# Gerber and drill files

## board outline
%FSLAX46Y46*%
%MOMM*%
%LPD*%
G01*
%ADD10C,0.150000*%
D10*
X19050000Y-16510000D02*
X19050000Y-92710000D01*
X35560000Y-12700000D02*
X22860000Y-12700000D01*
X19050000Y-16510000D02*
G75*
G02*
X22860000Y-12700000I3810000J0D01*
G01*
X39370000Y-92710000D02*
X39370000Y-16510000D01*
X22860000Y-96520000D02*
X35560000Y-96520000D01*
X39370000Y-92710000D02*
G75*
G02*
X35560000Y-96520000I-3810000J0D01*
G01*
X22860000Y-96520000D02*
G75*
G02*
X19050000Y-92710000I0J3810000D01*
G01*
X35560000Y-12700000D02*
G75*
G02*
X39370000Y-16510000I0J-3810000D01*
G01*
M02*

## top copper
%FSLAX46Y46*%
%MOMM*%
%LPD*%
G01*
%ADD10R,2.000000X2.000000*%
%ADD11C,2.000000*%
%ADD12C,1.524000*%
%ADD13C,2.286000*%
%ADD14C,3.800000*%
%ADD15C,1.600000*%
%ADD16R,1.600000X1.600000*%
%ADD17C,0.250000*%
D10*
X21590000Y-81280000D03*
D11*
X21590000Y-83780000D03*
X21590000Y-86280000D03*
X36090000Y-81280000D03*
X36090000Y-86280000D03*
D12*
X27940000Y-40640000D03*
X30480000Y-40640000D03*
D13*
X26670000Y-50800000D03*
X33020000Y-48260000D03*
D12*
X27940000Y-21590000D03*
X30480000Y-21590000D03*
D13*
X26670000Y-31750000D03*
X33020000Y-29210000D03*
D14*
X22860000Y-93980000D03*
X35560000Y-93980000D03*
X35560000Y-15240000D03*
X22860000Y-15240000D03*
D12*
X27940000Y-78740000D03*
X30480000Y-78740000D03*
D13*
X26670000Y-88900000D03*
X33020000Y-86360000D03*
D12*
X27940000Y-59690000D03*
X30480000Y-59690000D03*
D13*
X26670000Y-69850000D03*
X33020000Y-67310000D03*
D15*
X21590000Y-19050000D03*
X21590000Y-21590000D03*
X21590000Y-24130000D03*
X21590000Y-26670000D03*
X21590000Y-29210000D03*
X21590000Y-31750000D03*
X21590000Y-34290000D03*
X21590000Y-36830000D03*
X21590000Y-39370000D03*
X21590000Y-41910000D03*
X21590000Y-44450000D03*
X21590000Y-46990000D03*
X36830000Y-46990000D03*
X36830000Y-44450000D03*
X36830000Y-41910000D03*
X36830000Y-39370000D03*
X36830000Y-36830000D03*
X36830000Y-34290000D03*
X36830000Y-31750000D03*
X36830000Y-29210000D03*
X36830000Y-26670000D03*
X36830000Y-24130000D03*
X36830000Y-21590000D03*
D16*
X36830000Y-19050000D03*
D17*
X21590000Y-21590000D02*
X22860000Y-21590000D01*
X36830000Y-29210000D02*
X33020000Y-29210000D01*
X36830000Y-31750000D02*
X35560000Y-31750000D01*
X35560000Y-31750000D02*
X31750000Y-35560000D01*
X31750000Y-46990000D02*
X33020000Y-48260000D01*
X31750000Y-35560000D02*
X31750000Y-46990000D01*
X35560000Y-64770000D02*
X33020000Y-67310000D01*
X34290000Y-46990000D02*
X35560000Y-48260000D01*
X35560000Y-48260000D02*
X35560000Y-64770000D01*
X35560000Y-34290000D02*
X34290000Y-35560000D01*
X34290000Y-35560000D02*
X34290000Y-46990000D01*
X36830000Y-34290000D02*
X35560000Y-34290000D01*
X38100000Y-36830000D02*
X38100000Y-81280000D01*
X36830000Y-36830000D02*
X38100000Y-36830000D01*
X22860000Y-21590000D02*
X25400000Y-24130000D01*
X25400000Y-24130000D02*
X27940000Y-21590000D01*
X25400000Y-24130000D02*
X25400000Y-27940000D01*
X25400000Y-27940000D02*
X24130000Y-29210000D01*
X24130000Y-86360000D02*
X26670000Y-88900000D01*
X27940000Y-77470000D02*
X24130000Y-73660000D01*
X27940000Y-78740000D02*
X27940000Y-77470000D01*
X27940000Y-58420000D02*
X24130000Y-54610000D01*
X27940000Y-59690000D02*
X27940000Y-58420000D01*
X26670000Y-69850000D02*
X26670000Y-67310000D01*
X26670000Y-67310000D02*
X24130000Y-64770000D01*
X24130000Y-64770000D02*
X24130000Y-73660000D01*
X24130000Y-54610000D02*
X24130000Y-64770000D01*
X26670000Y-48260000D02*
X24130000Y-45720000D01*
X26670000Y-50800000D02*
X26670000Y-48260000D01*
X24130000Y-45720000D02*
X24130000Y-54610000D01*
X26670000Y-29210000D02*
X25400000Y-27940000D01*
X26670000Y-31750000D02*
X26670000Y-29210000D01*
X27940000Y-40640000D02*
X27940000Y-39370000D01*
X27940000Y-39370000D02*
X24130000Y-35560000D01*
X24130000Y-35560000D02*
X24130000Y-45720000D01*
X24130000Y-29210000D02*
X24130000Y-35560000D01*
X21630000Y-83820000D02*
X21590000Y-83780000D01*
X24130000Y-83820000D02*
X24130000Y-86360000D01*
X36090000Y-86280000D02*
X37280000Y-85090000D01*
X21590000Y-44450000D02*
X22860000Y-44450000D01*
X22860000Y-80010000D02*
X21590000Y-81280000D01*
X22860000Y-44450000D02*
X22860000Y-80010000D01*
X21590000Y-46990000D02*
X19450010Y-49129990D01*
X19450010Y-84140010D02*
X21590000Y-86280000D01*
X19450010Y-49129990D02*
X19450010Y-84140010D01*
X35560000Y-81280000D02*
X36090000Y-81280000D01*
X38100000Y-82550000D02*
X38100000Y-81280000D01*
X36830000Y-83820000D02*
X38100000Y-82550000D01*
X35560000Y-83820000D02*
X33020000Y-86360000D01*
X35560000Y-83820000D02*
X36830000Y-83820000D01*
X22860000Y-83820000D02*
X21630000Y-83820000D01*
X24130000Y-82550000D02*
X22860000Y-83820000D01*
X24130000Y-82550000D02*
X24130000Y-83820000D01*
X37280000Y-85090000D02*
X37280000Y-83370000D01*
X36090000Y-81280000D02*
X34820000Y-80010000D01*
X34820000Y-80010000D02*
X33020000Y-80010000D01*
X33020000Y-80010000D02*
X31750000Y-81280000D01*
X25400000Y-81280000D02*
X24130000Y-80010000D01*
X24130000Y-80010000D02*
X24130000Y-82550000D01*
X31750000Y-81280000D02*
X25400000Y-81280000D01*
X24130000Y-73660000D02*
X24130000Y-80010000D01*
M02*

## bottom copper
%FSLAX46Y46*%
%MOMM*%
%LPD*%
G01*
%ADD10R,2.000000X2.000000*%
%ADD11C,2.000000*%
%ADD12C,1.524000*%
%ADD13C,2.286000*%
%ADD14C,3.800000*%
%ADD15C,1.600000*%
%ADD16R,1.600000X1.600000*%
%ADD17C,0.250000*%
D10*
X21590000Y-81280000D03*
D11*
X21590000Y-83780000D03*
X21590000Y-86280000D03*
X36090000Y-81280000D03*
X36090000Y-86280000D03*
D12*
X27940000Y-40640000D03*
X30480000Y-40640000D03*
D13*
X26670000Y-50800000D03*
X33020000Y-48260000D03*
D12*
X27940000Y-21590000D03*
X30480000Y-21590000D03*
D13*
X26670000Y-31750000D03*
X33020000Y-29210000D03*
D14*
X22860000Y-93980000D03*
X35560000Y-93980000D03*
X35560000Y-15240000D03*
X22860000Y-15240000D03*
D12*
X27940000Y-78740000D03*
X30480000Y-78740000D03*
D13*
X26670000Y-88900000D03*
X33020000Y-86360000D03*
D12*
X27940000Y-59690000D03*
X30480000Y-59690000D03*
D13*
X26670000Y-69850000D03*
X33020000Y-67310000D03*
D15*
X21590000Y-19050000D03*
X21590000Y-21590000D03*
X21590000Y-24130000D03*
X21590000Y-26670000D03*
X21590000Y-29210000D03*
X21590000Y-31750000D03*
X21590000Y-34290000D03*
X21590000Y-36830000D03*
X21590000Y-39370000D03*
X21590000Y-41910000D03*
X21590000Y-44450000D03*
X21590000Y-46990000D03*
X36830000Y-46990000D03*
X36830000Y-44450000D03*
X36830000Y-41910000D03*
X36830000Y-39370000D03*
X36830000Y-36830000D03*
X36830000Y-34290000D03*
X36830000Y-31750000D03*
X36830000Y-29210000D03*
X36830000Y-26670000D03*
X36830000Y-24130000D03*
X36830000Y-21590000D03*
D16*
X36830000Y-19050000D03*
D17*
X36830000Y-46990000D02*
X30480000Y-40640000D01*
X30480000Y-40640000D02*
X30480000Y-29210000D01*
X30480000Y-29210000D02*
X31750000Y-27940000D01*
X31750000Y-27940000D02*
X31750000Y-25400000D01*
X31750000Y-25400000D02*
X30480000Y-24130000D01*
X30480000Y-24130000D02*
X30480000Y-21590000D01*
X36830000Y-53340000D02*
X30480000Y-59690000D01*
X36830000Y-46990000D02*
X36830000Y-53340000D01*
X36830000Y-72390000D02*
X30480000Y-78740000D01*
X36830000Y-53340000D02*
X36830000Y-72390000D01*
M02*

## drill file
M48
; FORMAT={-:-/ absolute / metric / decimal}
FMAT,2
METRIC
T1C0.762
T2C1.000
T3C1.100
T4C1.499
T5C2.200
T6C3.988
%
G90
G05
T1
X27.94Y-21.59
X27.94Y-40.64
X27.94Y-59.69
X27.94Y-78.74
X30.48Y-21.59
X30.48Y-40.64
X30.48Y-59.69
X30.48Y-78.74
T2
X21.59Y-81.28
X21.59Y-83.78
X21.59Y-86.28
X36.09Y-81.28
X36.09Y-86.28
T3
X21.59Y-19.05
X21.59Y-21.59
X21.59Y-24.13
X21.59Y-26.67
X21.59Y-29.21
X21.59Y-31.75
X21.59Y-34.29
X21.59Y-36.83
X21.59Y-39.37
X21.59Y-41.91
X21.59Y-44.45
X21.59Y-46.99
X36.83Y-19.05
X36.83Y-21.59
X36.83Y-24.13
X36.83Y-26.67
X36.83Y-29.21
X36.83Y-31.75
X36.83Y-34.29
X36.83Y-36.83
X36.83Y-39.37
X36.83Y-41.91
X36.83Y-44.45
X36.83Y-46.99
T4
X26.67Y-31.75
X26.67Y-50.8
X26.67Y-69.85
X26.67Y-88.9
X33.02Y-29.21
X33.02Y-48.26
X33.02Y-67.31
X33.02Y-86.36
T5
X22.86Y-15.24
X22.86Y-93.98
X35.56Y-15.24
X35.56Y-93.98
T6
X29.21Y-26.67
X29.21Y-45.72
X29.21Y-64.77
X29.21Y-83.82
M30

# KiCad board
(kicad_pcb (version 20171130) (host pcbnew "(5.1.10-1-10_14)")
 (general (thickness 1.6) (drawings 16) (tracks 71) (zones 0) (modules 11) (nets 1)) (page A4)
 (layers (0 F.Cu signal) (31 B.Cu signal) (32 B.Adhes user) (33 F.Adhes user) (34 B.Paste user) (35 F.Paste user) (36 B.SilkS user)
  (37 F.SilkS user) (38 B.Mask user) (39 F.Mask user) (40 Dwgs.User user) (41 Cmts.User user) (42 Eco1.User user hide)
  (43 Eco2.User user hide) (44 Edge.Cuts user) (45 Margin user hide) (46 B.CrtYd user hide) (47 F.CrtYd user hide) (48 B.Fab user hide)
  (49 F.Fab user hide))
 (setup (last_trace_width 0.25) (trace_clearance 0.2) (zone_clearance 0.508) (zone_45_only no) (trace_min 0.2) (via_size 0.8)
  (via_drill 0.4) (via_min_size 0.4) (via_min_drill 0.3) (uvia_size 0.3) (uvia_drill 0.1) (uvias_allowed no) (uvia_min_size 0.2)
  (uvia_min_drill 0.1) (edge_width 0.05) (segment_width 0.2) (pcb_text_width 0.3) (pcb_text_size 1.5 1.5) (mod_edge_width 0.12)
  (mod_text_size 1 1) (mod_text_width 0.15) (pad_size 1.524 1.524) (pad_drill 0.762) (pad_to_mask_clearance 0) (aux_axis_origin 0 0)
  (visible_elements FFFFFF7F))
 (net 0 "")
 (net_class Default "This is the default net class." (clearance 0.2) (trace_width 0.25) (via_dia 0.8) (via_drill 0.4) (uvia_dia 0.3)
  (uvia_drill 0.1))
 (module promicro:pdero (layer B.Cu) (at 27.94 57.15 180)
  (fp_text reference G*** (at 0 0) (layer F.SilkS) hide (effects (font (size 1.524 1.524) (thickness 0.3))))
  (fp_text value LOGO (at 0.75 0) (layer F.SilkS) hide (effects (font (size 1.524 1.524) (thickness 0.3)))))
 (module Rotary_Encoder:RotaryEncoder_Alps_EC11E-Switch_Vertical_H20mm (layer F.Cu) (at 21.59 81.28)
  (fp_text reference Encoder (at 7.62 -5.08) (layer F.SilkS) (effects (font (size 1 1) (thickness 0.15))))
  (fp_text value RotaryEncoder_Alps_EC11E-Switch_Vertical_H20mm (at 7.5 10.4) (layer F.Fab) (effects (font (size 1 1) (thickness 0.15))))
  (pad A thru_hole rect (at 0 0) (size 2 2) (drill 1) (layers *.Cu *.Mask))
  (pad C thru_hole circle (at 0 2.5) (size 2 2) (drill 1) (layers *.Cu *.Mask))
  (pad B thru_hole circle (at 0 5) (size 2 2) (drill 1) (layers *.Cu *.Mask))
  (pad S2 thru_hole circle (at 14.5 0) (size 2 2) (drill 1) (layers *.Cu *.Mask))
  (pad S1 thru_hole circle (at 14.5 5) (size 2 2) (drill 1) (layers *.Cu *.Mask)))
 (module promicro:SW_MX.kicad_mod (layer F.Cu) (at 29.21 45.72 180)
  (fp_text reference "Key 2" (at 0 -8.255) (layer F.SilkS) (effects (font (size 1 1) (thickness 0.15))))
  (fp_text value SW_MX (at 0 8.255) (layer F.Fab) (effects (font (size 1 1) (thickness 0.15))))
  (pad 4 thru_hole circle (at 1.27 5.08 180) (size 1.524 1.524) (drill 0.762) (layers *.Cu *.Mask))
  (pad 3 thru_hole circle (at -1.27 5.08 180) (size 1.524 1.524) (drill 0.762) (layers *.Cu *.Mask))
  (pad 1 thru_hole circle (at 2.54 -5.08 180) (size 2.286 2.286) (drill 1.4986) (layers *.Cu *.Mask))
  (pad "" np_thru_hole circle (at 0 0 180) (size 3.9878 3.9878) (drill 3.9878) (layers *.Cu *.Mask))
  (pad 2 thru_hole circle (at -3.81 -2.54 180) (size 2.286 2.286) (drill 1.4986) (layers *.Cu *.Mask)))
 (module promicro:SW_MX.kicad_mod (layer F.Cu) (at 29.21 26.67 180)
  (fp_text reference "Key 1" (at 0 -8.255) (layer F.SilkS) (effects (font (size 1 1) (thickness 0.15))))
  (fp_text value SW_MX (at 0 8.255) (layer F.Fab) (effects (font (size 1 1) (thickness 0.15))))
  (pad 4 thru_hole circle (at 1.27 5.08 180) (size 1.524 1.524) (drill 0.762) (layers *.Cu *.Mask))
  (pad 3 thru_hole circle (at -1.27 5.08 180) (size 1.524 1.524) (drill 0.762) (layers *.Cu *.Mask))
  (pad 1 thru_hole circle (at 2.54 -5.08 180) (size 2.286 2.286) (drill 1.4986) (layers *.Cu *.Mask))
  (pad "" np_thru_hole circle (at 0 0 180) (size 3.9878 3.9878) (drill 3.9878) (layers *.Cu *.Mask))
  (pad 2 thru_hole circle (at -3.81 -2.54 180) (size 2.286 2.286) (drill 1.4986) (layers *.Cu *.Mask)))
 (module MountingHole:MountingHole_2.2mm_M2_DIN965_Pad (layer F.Cu) (at 22.86 93.98)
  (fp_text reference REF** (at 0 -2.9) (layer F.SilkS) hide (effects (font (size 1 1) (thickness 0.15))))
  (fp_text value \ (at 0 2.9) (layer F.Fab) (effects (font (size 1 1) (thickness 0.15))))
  (pad 1 thru_hole circle (at 0 0) (size 3.8 3.8) (drill 2.2) (layers *.Cu *.Mask)))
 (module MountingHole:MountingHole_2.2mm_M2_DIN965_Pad (layer F.Cu) (at 35.56 93.98)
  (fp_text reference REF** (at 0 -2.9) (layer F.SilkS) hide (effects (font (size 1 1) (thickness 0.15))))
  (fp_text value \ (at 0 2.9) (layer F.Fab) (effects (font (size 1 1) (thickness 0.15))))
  (pad 1 thru_hole circle (at 0 0) (size 3.8 3.8) (drill 2.2) (layers *.Cu *.Mask)))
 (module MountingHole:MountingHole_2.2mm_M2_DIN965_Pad (layer F.Cu) (at 35.56 15.24)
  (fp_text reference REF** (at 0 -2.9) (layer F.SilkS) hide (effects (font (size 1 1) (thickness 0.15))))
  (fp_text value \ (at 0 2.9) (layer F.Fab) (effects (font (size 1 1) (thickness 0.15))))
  (pad 1 thru_hole circle (at 0 0) (size 3.8 3.8) (drill 2.2) (layers *.Cu *.Mask)))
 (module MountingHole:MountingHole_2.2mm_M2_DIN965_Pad (layer F.Cu) (at 22.86 15.24)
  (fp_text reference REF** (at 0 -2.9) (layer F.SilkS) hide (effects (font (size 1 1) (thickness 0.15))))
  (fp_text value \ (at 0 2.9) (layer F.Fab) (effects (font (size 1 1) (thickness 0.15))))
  (pad 1 thru_hole circle (at 0 0) (size 3.8 3.8) (drill 2.2) (layers *.Cu *.Mask)))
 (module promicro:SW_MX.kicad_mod (layer F.Cu) (at 29.21 83.82 180)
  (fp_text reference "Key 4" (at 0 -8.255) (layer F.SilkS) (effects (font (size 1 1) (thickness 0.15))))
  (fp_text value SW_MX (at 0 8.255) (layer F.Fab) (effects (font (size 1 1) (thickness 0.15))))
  (pad 4 thru_hole circle (at 1.27 5.08 180) (size 1.524 1.524) (drill 0.762) (layers *.Cu *.Mask))
  (pad 3 thru_hole circle (at -1.27 5.08 180) (size 1.524 1.524) (drill 0.762) (layers *.Cu *.Mask))
  (pad 1 thru_hole circle (at 2.54 -5.08 180) (size 2.286 2.286) (drill 1.4986) (layers *.Cu *.Mask))
  (pad "" np_thru_hole circle (at 0 0 180) (size 3.9878 3.9878) (drill 3.9878) (layers *.Cu *.Mask))
  (pad 2 thru_hole circle (at -3.81 -2.54 180) (size 2.286 2.286) (drill 1.4986) (layers *.Cu *.Mask)))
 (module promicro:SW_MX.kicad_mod (layer F.Cu) (at 29.21 64.77 180)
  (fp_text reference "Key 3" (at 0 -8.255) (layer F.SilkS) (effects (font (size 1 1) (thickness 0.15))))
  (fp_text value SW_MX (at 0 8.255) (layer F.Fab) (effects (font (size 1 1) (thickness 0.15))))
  (pad 4 thru_hole circle (at 1.27 5.08 180) (size 1.524 1.524) (drill 0.762) (layers *.Cu *.Mask))
  (pad 3 thru_hole circle (at -1.27 5.08 180) (size 1.524 1.524) (drill 0.762) (layers *.Cu *.Mask))
  (pad 1 thru_hole circle (at 2.54 -5.08 180) (size 2.286 2.286) (drill 1.4986) (layers *.Cu *.Mask))
  (pad "" np_thru_hole circle (at 0 0 180) (size 3.9878 3.9878) (drill 3.9878) (layers *.Cu *.Mask))
  (pad 2 thru_hole circle (at -3.81 -2.54 180) (size 2.286 2.286) (drill 1.4986) (layers *.Cu *.Mask)))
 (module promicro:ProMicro (layer B.Cu) (at 29.21 33.02 270)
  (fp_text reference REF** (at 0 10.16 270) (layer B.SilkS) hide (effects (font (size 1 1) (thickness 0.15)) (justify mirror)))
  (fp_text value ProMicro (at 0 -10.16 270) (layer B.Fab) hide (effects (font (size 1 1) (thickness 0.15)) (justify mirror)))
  (pad 24 thru_hole circle (at -13.97 7.62 270) (size 1.6 1.6) (drill 1.1) (layers *.Cu *.Mask B.SilkS))
  (pad 23 thru_hole circle (at -11.43 7.62 270) (size 1.6 1.6) (drill 1.1) (layers *.Cu *.Mask B.SilkS))
  (pad 22 thru_hole circle (at -8.89 7.62 270) (size 1.6 1.6) (drill 1.1) (layers *.Cu *.Mask B.SilkS))
  (pad 21 thru_hole circle (at -6.35 7.62 270) (size 1.6 1.6) (drill 1.1) (layers *.Cu *.Mask B.SilkS))
  (pad 20 thru_hole circle (at -3.81 7.62 270) (size 1.6 1.6) (drill 1.1) (layers *.Cu *.Mask B.SilkS))
  (pad 19 thru_hole circle (at -1.27 7.62 270) (size 1.6 1.6) (drill 1.1) (layers *.Cu *.Mask B.SilkS))
  (pad 18 thru_hole circle (at 1.27 7.62 270) (size 1.6 1.6) (drill 1.1) (layers *.Cu *.Mask B.SilkS))
  (pad 17 thru_hole circle (at 3.81 7.62 270) (size 1.6 1.6) (drill 1.1) (layers *.Cu *.Mask B.SilkS))
  (pad 16 thru_hole circle (at 6.35 7.62 270) (size 1.6 1.6) (drill 1.1) (layers *.Cu *.Mask B.SilkS))
  (pad 15 thru_hole circle (at 8.89 7.62 270) (size 1.6 1.6) (drill 1.1) (layers *.Cu *.Mask B.SilkS))
  (pad 14 thru_hole circle (at 11.43 7.62 270) (size 1.6 1.6) (drill 1.1) (layers *.Cu *.Mask B.SilkS))
  (pad 13 thru_hole circle (at 13.97 7.62 270) (size 1.6 1.6) (drill 1.1) (layers *.Cu *.Mask B.SilkS))
  (pad 12 thru_hole circle (at 13.97 -7.62 270) (size 1.6 1.6) (drill 1.1) (layers *.Cu *.Mask B.SilkS))
  (pad 11 thru_hole circle (at 11.43 -7.62 270) (size 1.6 1.6) (drill 1.1) (layers *.Cu *.Mask B.SilkS))
  (pad 10 thru_hole circle (at 8.89 -7.62 270) (size 1.6 1.6) (drill 1.1) (layers *.Cu *.Mask B.SilkS))
  (pad 9 thru_hole circle (at 6.35 -7.62 270) (size 1.6 1.6) (drill 1.1) (layers *.Cu *.Mask B.SilkS))
  (pad 8 thru_hole circle (at 3.81 -7.62 270) (size 1.6 1.6) (drill 1.1) (layers *.Cu *.Mask B.SilkS))
  (pad 7 thru_hole circle (at 1.27 -7.62 270) (size 1.6 1.6) (drill 1.1) (layers *.Cu *.Mask B.SilkS))
  (pad 6 thru_hole circle (at -1.27 -7.62 270) (size 1.6 1.6) (drill 1.1) (layers *.Cu *.Mask B.SilkS))
  (pad 5 thru_hole circle (at -3.81 -7.62 270) (size 1.6 1.6) (drill 1.1) (layers *.Cu *.Mask B.SilkS))
  (pad 4 thru_hole circle (at -6.35 -7.62 270) (size 1.6 1.6) (drill 1.1) (layers *.Cu *.Mask B.SilkS))
  (pad 3 thru_hole circle (at -8.89 -7.62 270) (size 1.6 1.6) (drill 1.1) (layers *.Cu *.Mask B.SilkS))
  (pad 2 thru_hole circle (at -11.43 -7.62 270) (size 1.6 1.6) (drill 1.1) (layers *.Cu *.Mask B.SilkS))
  (pad 1 thru_hole rect (at -13.97 -7.62 270) (size 1.6 1.6) (drill 1.1) (layers *.Cu *.Mask B.SilkS)))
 (gr_line (start 19.05 16.51) (end 19.05 92.71) (layer Edge.Cuts) (width 0.15))
 (gr_line (start 35.56 12.7) (end 22.86 12.7) (layer Edge.Cuts) (width 0.15))
 (gr_arc (start 22.86 16.51) (end 22.86 12.7) (angle -90) (layer Edge.Cuts) (width 0.15))
 (gr_line (start 39.37 92.71) (end 39.37 16.51) (layer Edge.Cuts) (width 0.15))
 (gr_line (start 22.86 96.52) (end 35.56 96.52) (layer Edge.Cuts) (width 0.15))
 (gr_arc (start 35.56 92.71) (end 35.56 96.52) (angle -90) (layer Edge.Cuts) (width 0.15))
 (gr_arc (start 22.86 92.71) (end 19.05 92.71) (angle -90) (layer Edge.Cuts) (width 0.15))
 (gr_arc (start 35.56 16.51) (end 39.37 16.51) (angle -90) (layer Edge.Cuts) (width 0.15))
 (segment (start 21.59 21.59) (end 22.86 21.59) (width 0.25) (layer F.Cu) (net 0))
 (segment (start 36.83 29.21) (end 33.02 29.21) (width 0.25) (layer F.Cu) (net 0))
 (segment (start 36.83 46.99) (end 30.48 40.64) (width 0.25) (layer B.Cu) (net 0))
 (segment (start 30.48 40.64) (end 30.48 29.21) (width 0.25) (layer B.Cu) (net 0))
 (segment (start 30.48 29.21) (end 31.75 27.94) (width 0.25) (layer B.Cu) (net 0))
 (segment (start 31.75 27.94) (end 31.75 25.4) (width 0.25) (layer B.Cu) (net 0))
 (segment (start 31.75 25.4) (end 30.48 24.13) (width 0.25) (layer B.Cu) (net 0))
 (segment (start 30.48 24.13) (end 30.48 21.59) (width 0.25) (layer B.Cu) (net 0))
 (segment (start 36.83 53.34) (end 30.48 59.69) (width 0.25) (layer B.Cu) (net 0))
 (segment (start 36.83 46.99) (end 36.83 53.34) (width 0.25) (layer B.Cu) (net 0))
 (segment (start 36.83 72.39) (end 30.48 78.74) (width 0.25) (layer B.Cu) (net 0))
 (segment (start 36.83 53.34) (end 36.83 72.39) (width 0.25) (layer B.Cu) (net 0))
 (segment (start 36.83 31.75) (end 35.56 31.75) (width 0.25) (layer F.Cu) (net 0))
 (segment (start 35.56 31.75) (end 31.75 35.56) (width 0.25) (layer F.Cu) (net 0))
 (segment (start 31.75 46.99) (end 33.02 48.26) (width 0.25) (layer F.Cu) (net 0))
 (segment (start 31.75 35.56) (end 31.75 46.99) (width 0.25) (layer F.Cu) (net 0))
 (segment (start 35.56 64.77) (end 33.02 67.31) (width 0.25) (layer F.Cu) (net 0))
 (segment (start 34.29 46.99) (end 35.56 48.26) (width 0.25) (layer F.Cu) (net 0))
 (segment (start 35.56 48.26) (end 35.56 64.77) (width 0.25) (layer F.Cu) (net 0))
 (segment (start 35.56 34.29) (end 34.29 35.56) (width 0.25) (layer F.Cu) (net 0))
 (segment (start 34.29 35.56) (end 34.29 46.99) (width 0.25) (layer F.Cu) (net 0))
 (segment (start 36.83 34.29) (end 35.56 34.29) (width 0.25) (layer F.Cu) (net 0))
 (segment (start 38.1 36.83) (end 38.1 81.28) (width 0.25) (layer F.Cu) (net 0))
 (segment (start 36.83 36.83) (end 38.1 36.83) (width 0.25) (layer F.Cu) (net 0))
 (segment (start 22.86 21.59) (end 25.4 24.13) (width 0.25) (layer F.Cu) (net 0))
 (segment (start 25.4 24.13) (end 27.94 21.59) (width 0.25) (layer F.Cu) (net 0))
 (segment (start 25.4 24.13) (end 25.4 27.94) (width 0.25) (layer F.Cu) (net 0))
 (segment (start 25.4 27.94) (end 24.13 29.21) (width 0.25) (layer F.Cu) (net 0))
 (segment (start 24.13 86.36) (end 26.67 88.9) (width 0.25) (layer F.Cu) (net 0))
 (segment (start 27.94 77.47) (end 24.13 73.66) (width 0.25) (layer F.Cu) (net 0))
 (segment (start 27.94 78.74) (end 27.94 77.47) (width 0.25) (layer F.Cu) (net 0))
 (segment (start 27.94 58.42) (end 24.13 54.61) (width 0.25) (layer F.Cu) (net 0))
 (segment (start 27.94 59.69) (end 27.94 58.42) (width 0.25) (layer F.Cu) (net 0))
 (segment (start 26.67 69.85) (end 26.67 67.31) (width 0.25) (layer F.Cu) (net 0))
 (segment (start 26.67 67.31) (end 24.13 64.77) (width 0.25) (layer F.Cu) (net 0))
 (segment (start 24.13 64.77) (end 24.13 73.66) (width 0.25) (layer F.Cu) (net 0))
 (segment (start 24.13 54.61) (end 24.13 64.77) (width 0.25) (layer F.Cu) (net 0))
 (segment (start 26.67 48.26) (end 24.13 45.72) (width 0.25) (layer F.Cu) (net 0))
 (segment (start 26.67 50.8) (end 26.67 48.26) (width 0.25) (layer F.Cu) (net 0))
 (segment (start 24.13 45.72) (end 24.13 54.61) (width 0.25) (layer F.Cu) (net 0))
 (segment (start 26.67 29.21) (end 25.4 27.94) (width 0.25) (layer F.Cu) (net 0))
 (segment (start 26.67 31.75) (end 26.67 29.21) (width 0.25) (layer F.Cu) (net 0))
 (segment (start 27.94 40.64) (end 27.94 39.37) (width 0.25) (layer F.Cu) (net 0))
 (segment (start 27.94 39.37) (end 24.13 35.56) (width 0.25) (layer F.Cu) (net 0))
 (segment (start 24.13 35.56) (end 24.13 45.72) (width 0.25) (layer F.Cu) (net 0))
 (segment (start 24.13 29.21) (end 24.13 35.56) (width 0.25) (layer F.Cu) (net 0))
 (segment (start 21.63 83.82) (end 21.59 83.78) (width 0.25) (layer F.Cu) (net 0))
 (segment (start 24.13 83.82) (end 24.13 86.36) (width 0.25) (layer F.Cu) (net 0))
 (segment (start 36.09 86.28) (end 37.28 85.09) (width 0.25) (layer F.Cu) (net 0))
 (segment (start 21.59 44.45) (end 22.86 44.45) (width 0.25) (layer F.Cu) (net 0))
 (segment (start 22.86 80.01) (end 21.59 81.28) (width 0.25) (layer F.Cu) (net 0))
 (segment (start 22.86 44.45) (end 22.86 80.01) (width 0.25) (layer F.Cu) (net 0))
 (segment (start 21.59 46.99) (end 19.45001 49.12999) (width 0.25) (layer F.Cu) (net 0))
 (segment (start 19.45001 84.14001) (end 21.59 86.28) (width 0.25) (layer F.Cu) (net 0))
 (segment (start 19.45001 49.12999) (end 19.45001 84.14001) (width 0.25) (layer F.Cu) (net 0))
 (segment (start 35.56 81.28) (end 36.09 81.28) (width 0.25) (layer F.Cu) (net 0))
 (segment (start 38.1 82.55) (end 38.1 81.28) (width 0.25) (layer F.Cu) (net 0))
 (segment (start 36.83 83.82) (end 38.1 82.55) (width 0.25) (layer F.Cu) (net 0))
 (segment (start 35.56 83.82) (end 33.02 86.36) (width 0.25) (layer F.Cu) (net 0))
 (segment (start 35.56 83.82) (end 36.83 83.82) (width 0.25) (layer F.Cu) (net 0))
 (segment (start 22.86 83.82) (end 21.63 83.82) (width 0.25) (layer F.Cu) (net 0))
 (segment (start 24.13 82.55) (end 22.86 83.82) (width 0.25) (layer F.Cu) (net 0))
 (segment (start 24.13 82.55) (end 24.13 83.82) (width 0.25) (layer F.Cu) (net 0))
 (segment (start 37.28 85.09) (end 37.28 83.37) (width 0.25) (layer F.Cu) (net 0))
 (segment (start 36.09 81.28) (end 34.82 80.01) (width 0.25) (layer F.Cu) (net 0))
 (segment (start 34.82 80.01) (end 33.02 80.01) (width 0.25) (layer F.Cu) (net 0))
 (segment (start 33.02 80.01) (end 31.75 81.28) (width 0.25) (layer F.Cu) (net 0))
 (segment (start 25.4 81.28) (end 24.13 80.01) (width 0.25) (layer F.Cu) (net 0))
 (segment (start 24.13 80.01) (end 24.13 82.55) (width 0.25) (layer F.Cu) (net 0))
 (segment (start 31.75 81.28) (end 25.4 81.28) (width 0.25) (layer F.Cu) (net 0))
 (segment (start 24.13 73.66) (end 24.13 80.01) (width 0.25) (layer F.Cu) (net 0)))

